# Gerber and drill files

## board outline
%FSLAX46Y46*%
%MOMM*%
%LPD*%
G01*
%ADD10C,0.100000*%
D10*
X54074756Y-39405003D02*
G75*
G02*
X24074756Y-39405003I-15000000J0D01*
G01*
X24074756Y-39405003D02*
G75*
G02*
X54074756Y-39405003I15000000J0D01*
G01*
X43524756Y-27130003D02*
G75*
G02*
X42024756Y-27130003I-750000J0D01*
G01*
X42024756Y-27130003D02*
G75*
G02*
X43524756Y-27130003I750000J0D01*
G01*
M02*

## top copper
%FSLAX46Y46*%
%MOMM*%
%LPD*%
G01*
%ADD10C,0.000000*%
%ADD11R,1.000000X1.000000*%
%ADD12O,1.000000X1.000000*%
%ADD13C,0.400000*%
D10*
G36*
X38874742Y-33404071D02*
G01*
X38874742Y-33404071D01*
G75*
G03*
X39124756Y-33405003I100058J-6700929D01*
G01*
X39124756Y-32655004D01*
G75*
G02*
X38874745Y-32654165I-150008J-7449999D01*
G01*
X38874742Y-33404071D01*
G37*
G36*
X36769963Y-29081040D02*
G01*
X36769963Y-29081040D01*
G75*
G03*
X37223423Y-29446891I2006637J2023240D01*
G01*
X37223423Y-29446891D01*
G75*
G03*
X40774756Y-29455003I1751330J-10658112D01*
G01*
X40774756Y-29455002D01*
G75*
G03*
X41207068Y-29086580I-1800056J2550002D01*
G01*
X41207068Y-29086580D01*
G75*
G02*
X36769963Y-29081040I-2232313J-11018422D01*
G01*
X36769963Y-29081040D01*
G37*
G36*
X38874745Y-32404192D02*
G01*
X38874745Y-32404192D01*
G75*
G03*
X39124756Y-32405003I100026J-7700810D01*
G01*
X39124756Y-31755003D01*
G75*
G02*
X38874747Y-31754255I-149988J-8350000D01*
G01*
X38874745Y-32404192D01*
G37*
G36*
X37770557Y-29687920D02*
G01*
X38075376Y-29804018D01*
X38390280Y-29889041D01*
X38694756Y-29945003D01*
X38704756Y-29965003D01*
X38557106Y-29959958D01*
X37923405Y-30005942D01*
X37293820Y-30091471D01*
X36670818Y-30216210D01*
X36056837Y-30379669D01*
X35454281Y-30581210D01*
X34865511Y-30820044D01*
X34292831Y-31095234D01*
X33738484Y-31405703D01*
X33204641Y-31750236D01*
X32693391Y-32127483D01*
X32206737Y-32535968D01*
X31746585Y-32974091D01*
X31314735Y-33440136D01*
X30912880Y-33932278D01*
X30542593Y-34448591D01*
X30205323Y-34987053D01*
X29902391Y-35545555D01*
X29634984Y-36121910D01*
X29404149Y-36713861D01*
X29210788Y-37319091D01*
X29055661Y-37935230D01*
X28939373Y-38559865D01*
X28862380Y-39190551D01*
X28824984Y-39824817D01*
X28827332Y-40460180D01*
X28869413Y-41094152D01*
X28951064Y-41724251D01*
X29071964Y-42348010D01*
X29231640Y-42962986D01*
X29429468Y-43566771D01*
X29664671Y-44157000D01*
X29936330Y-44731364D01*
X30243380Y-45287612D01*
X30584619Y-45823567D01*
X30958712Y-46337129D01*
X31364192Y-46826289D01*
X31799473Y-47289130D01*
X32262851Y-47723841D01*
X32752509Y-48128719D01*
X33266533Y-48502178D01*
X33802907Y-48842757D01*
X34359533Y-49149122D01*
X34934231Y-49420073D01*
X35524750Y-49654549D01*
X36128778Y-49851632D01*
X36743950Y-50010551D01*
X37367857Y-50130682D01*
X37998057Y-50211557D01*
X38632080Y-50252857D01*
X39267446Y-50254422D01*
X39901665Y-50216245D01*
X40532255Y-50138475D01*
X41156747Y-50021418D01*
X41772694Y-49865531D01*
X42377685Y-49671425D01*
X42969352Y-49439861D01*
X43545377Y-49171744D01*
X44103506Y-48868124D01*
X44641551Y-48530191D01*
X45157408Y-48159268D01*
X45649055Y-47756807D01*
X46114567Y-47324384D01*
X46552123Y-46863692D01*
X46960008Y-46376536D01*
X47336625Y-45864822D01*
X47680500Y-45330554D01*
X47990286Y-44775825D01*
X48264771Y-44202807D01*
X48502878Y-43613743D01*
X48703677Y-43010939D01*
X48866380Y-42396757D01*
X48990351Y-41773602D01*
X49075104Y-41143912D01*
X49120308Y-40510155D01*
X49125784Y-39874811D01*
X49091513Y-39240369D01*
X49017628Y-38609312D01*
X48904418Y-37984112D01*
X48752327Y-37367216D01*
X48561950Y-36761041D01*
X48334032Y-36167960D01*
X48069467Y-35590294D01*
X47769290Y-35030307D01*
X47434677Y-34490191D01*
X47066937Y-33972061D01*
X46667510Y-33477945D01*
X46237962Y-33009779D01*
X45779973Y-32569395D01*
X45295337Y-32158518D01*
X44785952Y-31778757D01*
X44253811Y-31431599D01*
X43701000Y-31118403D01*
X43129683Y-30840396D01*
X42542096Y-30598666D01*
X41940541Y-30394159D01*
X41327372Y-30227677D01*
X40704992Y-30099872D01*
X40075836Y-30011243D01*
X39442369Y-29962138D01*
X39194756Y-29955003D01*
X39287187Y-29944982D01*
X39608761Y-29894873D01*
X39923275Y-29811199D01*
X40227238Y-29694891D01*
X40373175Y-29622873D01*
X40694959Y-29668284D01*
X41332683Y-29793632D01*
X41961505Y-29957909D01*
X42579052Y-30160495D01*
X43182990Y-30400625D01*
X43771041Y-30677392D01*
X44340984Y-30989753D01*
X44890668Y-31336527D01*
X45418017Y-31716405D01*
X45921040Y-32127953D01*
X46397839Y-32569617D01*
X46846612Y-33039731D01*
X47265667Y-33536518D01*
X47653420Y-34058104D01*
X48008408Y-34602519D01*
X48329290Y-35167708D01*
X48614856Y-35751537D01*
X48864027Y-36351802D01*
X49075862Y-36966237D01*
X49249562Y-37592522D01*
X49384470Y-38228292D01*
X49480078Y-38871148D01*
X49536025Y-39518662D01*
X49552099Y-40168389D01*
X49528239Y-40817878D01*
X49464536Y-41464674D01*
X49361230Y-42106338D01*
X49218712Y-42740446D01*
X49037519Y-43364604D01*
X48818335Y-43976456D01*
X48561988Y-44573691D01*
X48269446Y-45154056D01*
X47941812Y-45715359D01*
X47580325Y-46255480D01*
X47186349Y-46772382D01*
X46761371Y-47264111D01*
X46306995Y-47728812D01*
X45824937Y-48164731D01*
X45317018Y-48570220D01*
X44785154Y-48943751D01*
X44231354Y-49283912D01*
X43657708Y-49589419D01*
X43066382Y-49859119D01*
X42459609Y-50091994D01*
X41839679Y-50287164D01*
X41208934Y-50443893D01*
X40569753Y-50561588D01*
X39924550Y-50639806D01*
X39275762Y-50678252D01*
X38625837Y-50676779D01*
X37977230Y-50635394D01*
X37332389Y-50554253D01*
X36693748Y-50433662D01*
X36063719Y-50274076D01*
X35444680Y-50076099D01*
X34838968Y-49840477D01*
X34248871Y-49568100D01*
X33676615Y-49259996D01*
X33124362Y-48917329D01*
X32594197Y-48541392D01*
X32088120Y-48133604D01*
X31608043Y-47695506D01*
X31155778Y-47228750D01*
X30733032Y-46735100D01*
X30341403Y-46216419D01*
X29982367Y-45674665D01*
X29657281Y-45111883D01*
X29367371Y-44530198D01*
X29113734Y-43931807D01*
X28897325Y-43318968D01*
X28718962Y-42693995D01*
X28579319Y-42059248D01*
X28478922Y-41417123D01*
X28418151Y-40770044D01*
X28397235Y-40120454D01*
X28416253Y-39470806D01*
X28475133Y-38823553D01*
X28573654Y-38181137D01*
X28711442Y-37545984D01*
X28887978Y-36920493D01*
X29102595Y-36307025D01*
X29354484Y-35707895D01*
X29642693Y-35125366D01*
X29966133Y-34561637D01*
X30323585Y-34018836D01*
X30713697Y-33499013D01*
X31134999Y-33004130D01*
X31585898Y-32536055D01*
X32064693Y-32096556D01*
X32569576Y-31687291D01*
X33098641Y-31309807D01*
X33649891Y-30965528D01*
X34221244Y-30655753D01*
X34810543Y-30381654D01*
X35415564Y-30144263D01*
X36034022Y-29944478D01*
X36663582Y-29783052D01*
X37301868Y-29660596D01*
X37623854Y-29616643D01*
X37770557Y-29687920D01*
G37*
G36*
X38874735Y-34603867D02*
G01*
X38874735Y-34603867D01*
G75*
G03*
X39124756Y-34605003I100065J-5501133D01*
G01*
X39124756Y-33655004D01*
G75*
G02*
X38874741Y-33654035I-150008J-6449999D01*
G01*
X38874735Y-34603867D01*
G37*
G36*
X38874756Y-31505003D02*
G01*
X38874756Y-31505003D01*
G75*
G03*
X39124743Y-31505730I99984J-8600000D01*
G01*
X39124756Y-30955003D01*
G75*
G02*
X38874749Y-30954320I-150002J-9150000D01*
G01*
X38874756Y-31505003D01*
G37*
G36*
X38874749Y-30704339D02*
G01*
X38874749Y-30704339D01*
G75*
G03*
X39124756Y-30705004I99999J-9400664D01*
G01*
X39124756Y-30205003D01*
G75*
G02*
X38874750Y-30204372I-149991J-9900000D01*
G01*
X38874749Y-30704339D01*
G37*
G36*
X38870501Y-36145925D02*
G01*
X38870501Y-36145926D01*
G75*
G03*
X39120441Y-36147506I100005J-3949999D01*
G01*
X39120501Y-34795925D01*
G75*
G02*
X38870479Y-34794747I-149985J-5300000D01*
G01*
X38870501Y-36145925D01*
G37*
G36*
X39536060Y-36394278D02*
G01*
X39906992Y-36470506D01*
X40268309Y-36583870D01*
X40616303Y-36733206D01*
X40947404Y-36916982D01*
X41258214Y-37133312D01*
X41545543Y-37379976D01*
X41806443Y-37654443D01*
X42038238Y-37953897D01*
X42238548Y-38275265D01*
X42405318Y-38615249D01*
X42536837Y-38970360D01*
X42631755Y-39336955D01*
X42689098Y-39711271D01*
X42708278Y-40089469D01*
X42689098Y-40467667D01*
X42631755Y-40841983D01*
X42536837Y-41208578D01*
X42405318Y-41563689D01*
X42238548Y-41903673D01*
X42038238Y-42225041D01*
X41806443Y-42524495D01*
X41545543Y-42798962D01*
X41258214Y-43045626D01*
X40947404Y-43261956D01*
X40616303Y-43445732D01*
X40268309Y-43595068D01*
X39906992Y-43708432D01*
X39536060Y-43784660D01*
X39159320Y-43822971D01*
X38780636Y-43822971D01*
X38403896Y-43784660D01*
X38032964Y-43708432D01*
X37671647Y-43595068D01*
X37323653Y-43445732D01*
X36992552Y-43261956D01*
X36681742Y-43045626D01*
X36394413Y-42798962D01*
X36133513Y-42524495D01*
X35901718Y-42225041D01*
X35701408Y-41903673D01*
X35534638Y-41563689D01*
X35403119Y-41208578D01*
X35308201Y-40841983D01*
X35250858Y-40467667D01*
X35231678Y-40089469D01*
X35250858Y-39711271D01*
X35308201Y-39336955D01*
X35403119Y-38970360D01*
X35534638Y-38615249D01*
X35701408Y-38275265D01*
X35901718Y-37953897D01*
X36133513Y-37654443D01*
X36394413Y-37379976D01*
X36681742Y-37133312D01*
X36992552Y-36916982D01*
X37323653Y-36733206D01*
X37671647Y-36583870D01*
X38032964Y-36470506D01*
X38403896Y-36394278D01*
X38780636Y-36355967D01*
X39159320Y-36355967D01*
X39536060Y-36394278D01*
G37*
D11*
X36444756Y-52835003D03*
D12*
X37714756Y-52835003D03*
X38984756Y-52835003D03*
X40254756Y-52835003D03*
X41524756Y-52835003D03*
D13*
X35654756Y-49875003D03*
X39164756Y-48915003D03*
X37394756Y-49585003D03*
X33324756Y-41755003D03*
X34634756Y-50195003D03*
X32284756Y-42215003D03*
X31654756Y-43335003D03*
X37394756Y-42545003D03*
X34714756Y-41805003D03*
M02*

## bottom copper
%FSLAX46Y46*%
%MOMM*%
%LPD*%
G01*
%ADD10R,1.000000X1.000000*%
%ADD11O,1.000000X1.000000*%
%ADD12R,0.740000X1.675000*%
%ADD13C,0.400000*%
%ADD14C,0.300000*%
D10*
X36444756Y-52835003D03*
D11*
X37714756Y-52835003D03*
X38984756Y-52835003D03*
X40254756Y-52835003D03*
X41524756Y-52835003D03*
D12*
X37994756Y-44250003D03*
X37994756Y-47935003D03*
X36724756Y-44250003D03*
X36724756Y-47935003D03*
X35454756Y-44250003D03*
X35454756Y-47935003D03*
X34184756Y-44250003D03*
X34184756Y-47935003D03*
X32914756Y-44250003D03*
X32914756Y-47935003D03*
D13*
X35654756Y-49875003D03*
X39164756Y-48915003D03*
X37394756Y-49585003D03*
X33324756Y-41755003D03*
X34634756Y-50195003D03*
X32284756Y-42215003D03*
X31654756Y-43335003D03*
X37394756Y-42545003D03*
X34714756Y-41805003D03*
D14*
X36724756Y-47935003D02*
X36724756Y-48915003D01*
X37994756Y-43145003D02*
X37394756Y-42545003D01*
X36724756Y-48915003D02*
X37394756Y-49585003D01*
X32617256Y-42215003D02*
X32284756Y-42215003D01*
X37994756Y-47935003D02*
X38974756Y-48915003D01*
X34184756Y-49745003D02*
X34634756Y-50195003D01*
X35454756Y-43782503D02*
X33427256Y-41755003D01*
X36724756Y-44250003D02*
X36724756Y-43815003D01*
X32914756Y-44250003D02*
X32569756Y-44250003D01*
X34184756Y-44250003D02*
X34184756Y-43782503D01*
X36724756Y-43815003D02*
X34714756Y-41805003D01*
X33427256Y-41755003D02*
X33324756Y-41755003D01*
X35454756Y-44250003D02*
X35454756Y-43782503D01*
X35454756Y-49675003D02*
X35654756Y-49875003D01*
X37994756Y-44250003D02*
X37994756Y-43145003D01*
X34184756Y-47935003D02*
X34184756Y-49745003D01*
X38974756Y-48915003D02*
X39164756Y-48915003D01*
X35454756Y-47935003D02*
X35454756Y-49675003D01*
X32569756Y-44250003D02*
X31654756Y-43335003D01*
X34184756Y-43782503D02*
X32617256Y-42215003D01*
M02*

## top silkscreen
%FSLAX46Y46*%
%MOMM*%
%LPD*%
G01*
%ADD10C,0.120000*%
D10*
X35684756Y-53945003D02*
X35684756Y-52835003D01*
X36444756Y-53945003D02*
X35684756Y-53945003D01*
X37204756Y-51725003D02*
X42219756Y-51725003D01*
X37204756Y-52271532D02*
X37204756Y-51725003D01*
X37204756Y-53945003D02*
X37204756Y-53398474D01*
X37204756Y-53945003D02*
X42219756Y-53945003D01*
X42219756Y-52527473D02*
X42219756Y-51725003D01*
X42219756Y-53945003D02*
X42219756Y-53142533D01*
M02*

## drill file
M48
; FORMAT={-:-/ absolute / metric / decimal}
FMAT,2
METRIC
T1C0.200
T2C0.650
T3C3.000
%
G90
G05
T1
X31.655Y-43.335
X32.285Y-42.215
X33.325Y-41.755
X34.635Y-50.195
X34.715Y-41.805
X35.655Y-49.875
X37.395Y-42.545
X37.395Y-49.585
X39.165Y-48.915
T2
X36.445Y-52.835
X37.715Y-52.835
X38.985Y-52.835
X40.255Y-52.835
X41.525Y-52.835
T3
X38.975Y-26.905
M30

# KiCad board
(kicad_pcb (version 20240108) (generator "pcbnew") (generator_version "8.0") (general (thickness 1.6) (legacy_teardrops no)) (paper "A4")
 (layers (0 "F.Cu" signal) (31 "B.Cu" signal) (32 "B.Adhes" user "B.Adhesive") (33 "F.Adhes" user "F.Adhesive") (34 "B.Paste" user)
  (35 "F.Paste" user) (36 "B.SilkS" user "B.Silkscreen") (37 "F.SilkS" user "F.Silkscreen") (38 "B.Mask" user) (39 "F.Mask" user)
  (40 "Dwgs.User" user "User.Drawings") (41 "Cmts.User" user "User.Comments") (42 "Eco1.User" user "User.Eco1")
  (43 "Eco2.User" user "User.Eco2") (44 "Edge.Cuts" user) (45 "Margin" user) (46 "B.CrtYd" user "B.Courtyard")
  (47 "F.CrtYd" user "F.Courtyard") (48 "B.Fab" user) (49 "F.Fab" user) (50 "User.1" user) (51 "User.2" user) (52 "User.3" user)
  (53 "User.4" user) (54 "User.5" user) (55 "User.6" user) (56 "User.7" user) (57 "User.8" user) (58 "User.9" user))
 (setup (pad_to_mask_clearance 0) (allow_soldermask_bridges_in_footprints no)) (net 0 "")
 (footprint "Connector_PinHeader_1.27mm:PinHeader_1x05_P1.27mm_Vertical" (layer "F.Cu") (at 36.444756 52.835003 90)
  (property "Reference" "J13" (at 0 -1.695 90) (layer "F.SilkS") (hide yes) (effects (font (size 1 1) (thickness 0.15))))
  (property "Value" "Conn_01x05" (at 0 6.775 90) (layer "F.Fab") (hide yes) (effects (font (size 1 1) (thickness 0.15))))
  (fp_line (start -1.11 -0.76) (end 0 -0.76) (stroke (width 0.12) (type solid)) (layer "F.SilkS"))
  (fp_line (start -1.11 0) (end -1.11 -0.76) (stroke (width 0.12) (type solid)) (layer "F.SilkS"))
  (fp_line (start 1.11 0.76) (end 1.11 5.775) (stroke (width 0.12) (type solid)) (layer "F.SilkS"))
  (fp_line (start 0.563471 0.76) (end 1.11 0.76) (stroke (width 0.12) (type solid)) (layer "F.SilkS"))
  (fp_line (start -1.11 0.76) (end -0.563471 0.76) (stroke (width 0.12) (type solid)) (layer "F.SilkS"))
  (fp_line (start -1.11 0.76) (end -1.11 5.775) (stroke (width 0.12) (type solid)) (layer "F.SilkS"))
  (fp_line (start 0.30753 5.775) (end 1.11 5.775) (stroke (width 0.12) (type solid)) (layer "F.SilkS"))
  (fp_line (start -1.11 5.775) (end -0.30753 5.775) (stroke (width 0.12) (type solid)) (layer "F.SilkS"))
  (pad "1" thru_hole rect (at 0 0 90) (size 1 1) (drill 0.65) (layers "*.Cu" "*.Mask") (remove_unused_layers no))
  (pad "2" thru_hole oval (at 0 1.27 90) (size 1 1) (drill 0.65) (layers "*.Cu" "*.Mask") (remove_unused_layers no))
  (pad "3" thru_hole oval (at 0 2.54 90) (size 1 1) (drill 0.65) (layers "*.Cu" "*.Mask") (remove_unused_layers no))
  (pad "4" thru_hole oval (at 0 3.81 90) (size 1 1) (drill 0.65) (layers "*.Cu" "*.Mask") (remove_unused_layers no))
  (pad "5" thru_hole oval (at 0 5.08 90) (size 1 1) (drill 0.65) (layers "*.Cu" "*.Mask") (remove_unused_layers no)))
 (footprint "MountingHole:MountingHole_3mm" (layer "F.Cu") (at 38.974756 26.905003)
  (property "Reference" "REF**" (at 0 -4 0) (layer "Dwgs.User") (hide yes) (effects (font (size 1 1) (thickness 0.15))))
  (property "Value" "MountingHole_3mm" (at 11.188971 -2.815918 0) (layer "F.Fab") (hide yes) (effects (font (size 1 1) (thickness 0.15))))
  (pad "" np_thru_hole circle (at 0 0) (size 3 3) (drill 3) (layers "*.Cu" "*.Mask")))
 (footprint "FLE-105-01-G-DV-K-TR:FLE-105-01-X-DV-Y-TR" (layer "B.Cu") (at 35.454756 46.092503 180)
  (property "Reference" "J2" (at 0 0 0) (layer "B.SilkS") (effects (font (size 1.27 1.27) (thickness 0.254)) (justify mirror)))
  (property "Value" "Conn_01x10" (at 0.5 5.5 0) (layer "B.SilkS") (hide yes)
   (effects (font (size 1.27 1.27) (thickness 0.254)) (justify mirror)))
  (pad "1" smd rect (at -2.54 1.8425 180) (size 0.74 1.675) (layers "B.Cu" "B.Paste" "B.Mask"))
  (pad "2" smd rect (at -2.54 -1.8425 180) (size 0.74 1.675) (layers "B.Cu" "B.Paste" "B.Mask"))
  (pad "3" smd rect (at -1.27 1.8425 180) (size 0.74 1.675) (layers "B.Cu" "B.Paste" "B.Mask"))
  (pad "4" smd rect (at -1.27 -1.8425 180) (size 0.74 1.675) (layers "B.Cu" "B.Paste" "B.Mask"))
  (pad "5" smd rect (at 0 1.8425 180) (size 0.74 1.675) (layers "B.Cu" "B.Paste" "B.Mask"))
  (pad "6" smd rect (at 0 -1.8425 180) (size 0.74 1.675) (layers "B.Cu" "B.Paste" "B.Mask"))
  (pad "7" smd rect (at 1.27 1.8425 180) (size 0.74 1.675) (layers "B.Cu" "B.Paste" "B.Mask"))
  (pad "8" smd rect (at 1.27 -1.8425 180) (size 0.74 1.675) (layers "B.Cu" "B.Paste" "B.Mask"))
  (pad "9" smd rect (at 2.54 1.8425 180) (size 0.74 1.675) (layers "B.Cu" "B.Paste" "B.Mask"))
  (pad "10" smd rect (at 2.54 -1.8425 180) (size 0.74 1.675) (layers "B.Cu" "B.Paste" "B.Mask")))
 (gr_poly
  (pts
   (arc (start 38.874745 32.654165) (mid 38.949758 47.55647) (end 39.124756 32.655004))
   (arc (start 39.124756 33.405003) (mid 38.949789 46.806633) (end 38.874742 33.404071)))
  (stroke (width 0) (type solid)) (fill solid) (layer "F.Cu"))
 (gr_poly
  (pts
   (arc (start 37.223423 29.446891) (mid 38.950087 50.906016) (end 40.774756 29.455003))
   (arc (start 40.774756 29.455002) (mid 40.99931 29.280645) (end 41.207068 29.08658))
   (arc (start 41.207068 29.08658) (mid 38.960716 51.347273) (end 36.769963 29.08104))
   (arc (start 36.769963 29.08104) (mid 36.987318 29.275586) (end 37.223423 29.446891)))
  (stroke (width 0) (type solid)) (fill solid) (layer "F.Cu"))
 (gr_poly
  (pts
   (arc (start 38.874745 32.404192) (mid 38.949788 47.806421) (end 39.124756 32.405003))
   (arc (start 39.124756 31.755003) (mid 38.949758 48.456313) (end 38.874747 31.754255)))
  (stroke (width 0) (type solid)) (fill solid) (layer "F.Cu"))
 (gr_poly
  (pts (xy 39.194756 29.955003) (xy 39.287187 29.944982) (xy 39.608761 29.894873) (xy 39.923275 29.811199) (xy 40.227238 29.694891)
   (xy 40.373175 29.622873) (xy 40.694959 29.668284) (xy 41.332683 29.793632) (xy 41.961505 29.957909) (xy 42.579052 30.160495)
   (xy 43.18299 30.400625) (xy 43.771041 30.677392) (xy 44.340984 30.989753) (xy 44.890668 31.336527) (xy 45.418017 31.716405)
   (xy 45.92104 32.127953) (xy 46.397839 32.569617) (xy 46.846612 33.039731) (xy 47.265667 33.536518) (xy 47.65342 34.058104)
   (xy 48.008408 34.602519) (xy 48.32929 35.167708) (xy 48.614856 35.751537) (xy 48.864027 36.351802) (xy 49.075862 36.966237)
   (xy 49.249562 37.592522) (xy 49.38447 38.228292) (xy 49.480078 38.871148) (xy 49.536025 39.518662) (xy 49.552099 40.168389)
   (xy 49.528239 40.817878) (xy 49.464536 41.464674) (xy 49.36123 42.106338) (xy 49.218712 42.740446) (xy 49.037519 43.364604)
   (xy 48.818335 43.976456) (xy 48.561988 44.573691) (xy 48.269446 45.154056) (xy 47.941812 45.715359) (xy 47.580325 46.25548)
   (xy 47.186349 46.772382) (xy 46.761371 47.264111) (xy 46.306995 47.728812) (xy 45.824937 48.164731) (xy 45.317018 48.57022)
   (xy 44.785154 48.943751) (xy 44.231354 49.283912) (xy 43.657708 49.589419) (xy 43.066382 49.859119) (xy 42.459609 50.091994)
   (xy 41.839679 50.287164) (xy 41.208934 50.443893) (xy 40.569753 50.561588) (xy 39.92455 50.639806) (xy 39.275762 50.678252)
   (xy 38.625837 50.676779) (xy 37.97723 50.635394) (xy 37.332389 50.554253) (xy 36.693748 50.433662) (xy 36.063719 50.274076)
   (xy 35.44468 50.076099) (xy 34.838968 49.840477) (xy 34.248871 49.5681) (xy 33.676615 49.259996) (xy 33.124362 48.917329)
   (xy 32.594197 48.541392) (xy 32.08812 48.133604) (xy 31.608043 47.695506) (xy 31.155778 47.22875) (xy 30.733032 46.7351)
   (xy 30.341403 46.216419) (xy 29.982367 45.674665) (xy 29.657281 45.111883) (xy 29.367371 44.530198) (xy 29.113734 43.931807)
   (xy 28.897325 43.318968) (xy 28.718962 42.693995) (xy 28.579319 42.059248) (xy 28.478922 41.417123) (xy 28.418151 40.770044)
   (xy 28.397235 40.120454) (xy 28.416253 39.470806) (xy 28.475133 38.823553) (xy 28.573654 38.181137) (xy 28.711442 37.545984)
   (xy 28.887978 36.920493) (xy 29.102595 36.307025) (xy 29.354484 35.707895) (xy 29.642693 35.125366) (xy 29.966133 34.561637)
   (xy 30.323585 34.018836) (xy 30.713697 33.499013) (xy 31.134999 33.00413) (xy 31.585898 32.536055) (xy 32.064693 32.096556)
   (xy 32.569576 31.687291) (xy 33.098641 31.309807) (xy 33.649891 30.965528) (xy 34.221244 30.655753) (xy 34.810543 30.381654)
   (xy 35.415564 30.144263) (xy 36.034022 29.944478) (xy 36.663582 29.783052) (xy 37.301868 29.660596) (xy 37.623854 29.616643)
   (xy 37.770557 29.68792) (xy 38.075376 29.804018) (xy 38.39028 29.889041) (xy 38.694756 29.945003) (xy 38.704756 29.965003)
   (xy 38.557106 29.959958) (xy 37.923405 30.005942) (xy 37.29382 30.091471) (xy 36.670818 30.21621) (xy 36.056837 30.379669)
   (xy 35.454281 30.58121) (xy 34.865511 30.820044) (xy 34.292831 31.095234) (xy 33.738484 31.405703) (xy 33.204641 31.750236)
   (xy 32.693391 32.127483) (xy 32.206737 32.535968) (xy 31.746585 32.974091) (xy 31.314735 33.440136) (xy 30.91288 33.932278)
   (xy 30.542593 34.448591) (xy 30.205323 34.987053) (xy 29.902391 35.545555) (xy 29.634984 36.12191) (xy 29.404149 36.713861)
   (xy 29.210788 37.319091) (xy 29.055661 37.93523) (xy 28.939373 38.559865) (xy 28.86238 39.190551) (xy 28.824984 39.824817)
   (xy 28.827332 40.46018) (xy 28.869413 41.094152) (xy 28.951064 41.724251) (xy 29.071964 42.34801) (xy 29.23164 42.962986)
   (xy 29.429468 43.566771) (xy 29.664671 44.157) (xy 29.93633 44.731364) (xy 30.24338 45.287612) (xy 30.584619 45.823567)
   (xy 30.958712 46.337129) (xy 31.364192 46.826289) (xy 31.799473 47.28913) (xy 32.262851 47.723841) (xy 32.752509 48.128719)
   (xy 33.266533 48.502178) (xy 33.802907 48.842757) (xy 34.359533 49.149122) (xy 34.934231 49.420073) (xy 35.52475 49.654549)
   (xy 36.128778 49.851632) (xy 36.74395 50.010551) (xy 37.367857 50.130682) (xy 37.998057 50.211557) (xy 38.63208 50.252857)
   (xy 39.267446 50.254422) (xy 39.901665 50.216245) (xy 40.532255 50.138475) (xy 41.156747 50.021418) (xy 41.772694 49.865531)
   (xy 42.377685 49.671425) (xy 42.969352 49.439861) (xy 43.545377 49.171744) (xy 44.103506 48.868124) (xy 44.641551 48.530191)
   (xy 45.157408 48.159268) (xy 45.649055 47.756807) (xy 46.114567 47.324384) (xy 46.552123 46.863692) (xy 46.960008 46.376536)
   (xy 47.336625 45.864822) (xy 47.6805 45.330554) (xy 47.990286 44.775825) (xy 48.264771 44.202807) (xy 48.502878 43.613743)
   (xy 48.703677 43.010939) (xy 48.86638 42.396757) (xy 48.990351 41.773602) (xy 49.075104 41.143912) (xy 49.120308 40.510155)
   (xy 49.125784 39.874811) (xy 49.091513 39.240369) (xy 49.017628 38.609312) (xy 48.904418 37.984112) (xy 48.752327 37.367216)
   (xy 48.56195 36.761041) (xy 48.334032 36.16796) (xy 48.069467 35.590294) (xy 47.76929 35.030307) (xy 47.434677 34.490191)
   (xy 47.066937 33.972061) (xy 46.66751 33.477945) (xy 46.237962 33.009779) (xy 45.779973 32.569395) (xy 45.295337 32.158518)
   (xy 44.785952 31.778757) (xy 44.253811 31.431599) (xy 43.701 31.118403) (xy 43.129683 30.840396) (xy 42.542096 30.598666)
   (xy 41.940541 30.394159) (xy 41.327372 30.227677) (xy 40.704992 30.099872) (xy 40.075836 30.011243) (xy 39.442369 29.962138))
  (stroke (width 0) (type solid)) (fill solid) (layer "F.Cu"))
 (gr_poly
  (pts (xy 39.124756 33.655003)
   (arc (start 39.124756 34.605003) (mid 38.94976 45.606991) (end 38.874735 34.603867))
   (arc (start 38.874741 33.654035) (mid 38.949759 46.556698) (end 39.124756 33.655004)))
  (stroke (width 0) (type solid)) (fill solid) (layer "F.Cu"))
 (gr_poly
  (pts
   (arc (start 38.874756 31.505003) (mid 38.94976 48.705548) (end 39.124743 31.50573))
   (arc (start 39.124756 30.955003) (mid 38.949757 49.256198) (end 38.874749 30.95432)))
  (stroke (width 0) (type solid)) (fill solid) (layer "F.Cu"))
 (gr_poly
  (pts
   (arc (start 38.874749 30.704339) (mid 38.949757 49.506165) (end 39.124756 30.705004))
   (arc (start 39.124756 30.205003) (mid 38.949757 50.006108) (end 38.87475 30.204372)))
  (stroke (width 0) (type solid)) (fill solid) (layer "F.Cu"))
 (gr_poly
  (pts
   (arc (start 38.870501 36.145926) (mid 38.945519 44.047111) (end 39.120441 36.147506))
   (arc (start 39.120501 34.795925) (mid 38.945505 45.397988) (end 38.870479 34.794747)) (xy 38.870501 36.145925))
  (stroke (width 0) (type solid)) (fill solid) (layer "F.Cu"))
 (gr_poly
  (pts (xy 42.708278 40.089469) (xy 42.689098 39.711271) (xy 42.631755 39.336955) (xy 42.536837 38.97036) (xy 42.405318 38.615249)
   (xy 42.238548 38.275265) (xy 42.038238 37.953897) (xy 41.806443 37.654443) (xy 41.545543 37.379976) (xy 41.258214 37.133312)
   (xy 40.947404 36.916982) (xy 40.616303 36.733206) (xy 40.268309 36.58387) (xy 39.906992 36.470506) (xy 39.53606 36.394278)
   (xy 39.15932 36.355967) (xy 38.780636 36.355967) (xy 38.403896 36.394278) (xy 38.032964 36.470506) (xy 37.671647 36.58387)
   (xy 37.323653 36.733206) (xy 36.992552 36.916982) (xy 36.681742 37.133312) (xy 36.394413 37.379976) (xy 36.133513 37.654443)
   (xy 35.901718 37.953897) (xy 35.701408 38.275265) (xy 35.534638 38.615249) (xy 35.403119 38.97036) (xy 35.308201 39.336955)
   (xy 35.250858 39.711271) (xy 35.231678 40.089469) (xy 35.250858 40.467667) (xy 35.308201 40.841983) (xy 35.403119 41.208578)
   (xy 35.534638 41.563689) (xy 35.701408 41.903673) (xy 35.901718 42.225041) (xy 36.133513 42.524495) (xy 36.394413 42.798962)
   (xy 36.681742 43.045626) (xy 36.992552 43.261956) (xy 37.323653 43.445732) (xy 37.671647 43.595068) (xy 38.032964 43.708432)
   (xy 38.403896 43.78466) (xy 38.780636 43.822971) (xy 39.15932 43.822971) (xy 39.53606 43.78466) (xy 39.906992 43.708432)
   (xy 40.268309 43.595068) (xy 40.616303 43.445732) (xy 40.947404 43.261956) (xy 41.258214 43.045626) (xy 41.545543 42.798962)
   (xy 41.806443 42.524495) (xy 42.038238 42.225041) (xy 42.238548 41.903673) (xy 42.405318 41.563689) (xy 42.536837 41.208578)
   (xy 42.631755 40.841983) (xy 42.689098 40.467667) (xy 42.708278 40.089469))
  (stroke (width 0) (type solid)) (fill solid) (layer "F.Cu"))
 (gr_circle (center 39.074756 39.405003) (end 54.074756 39.405003) (stroke (width 0.1) (type default)) (fill none) (layer "Edge.Cuts"))
 (gr_circle (center 42.774756 27.130003) (end 43.524756 27.130003) (stroke (width 0.1) (type default)) (fill none) (layer "Edge.Cuts"))
 (via (at 35.654756 49.875003) (size 0.4) (drill 0.2) (layers "F.Cu" "B.Cu") (remove_unused_layers yes) (keep_end_layers yes)
  (zone_layer_connections) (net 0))
 (via (at 39.164756 48.915003) (size 0.4) (drill 0.2) (layers "F.Cu" "B.Cu") (remove_unused_layers yes) (keep_end_layers yes)
  (zone_layer_connections) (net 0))
 (via (at 37.394756 49.585003) (size 0.4) (drill 0.2) (layers "F.Cu" "B.Cu") (remove_unused_layers yes) (keep_end_layers yes)
  (zone_layer_connections) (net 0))
 (via (at 33.324756 41.755003) (size 0.4) (drill 0.2) (layers "F.Cu" "B.Cu") (remove_unused_layers yes) (keep_end_layers yes)
  (zone_layer_connections) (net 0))
 (via (at 34.634756 50.195003) (size 0.4) (drill 0.2) (layers "F.Cu" "B.Cu") (remove_unused_layers yes) (keep_end_layers yes)
  (zone_layer_connections) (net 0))
 (via (at 32.284756 42.215003) (size 0.4) (drill 0.2) (layers "F.Cu" "B.Cu") (remove_unused_layers yes) (keep_end_layers yes)
  (zone_layer_connections) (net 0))
 (via (at 31.654756 43.335003) (size 0.4) (drill 0.2) (layers "F.Cu" "B.Cu") (remove_unused_layers yes) (keep_end_layers yes)
  (zone_layer_connections) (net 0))
 (via (at 37.394756 42.545003) (size 0.4) (drill 0.2) (layers "F.Cu" "B.Cu") (remove_unused_layers yes) (keep_end_layers yes)
  (zone_layer_connections) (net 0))
 (via (at 34.714756 41.805003) (size 0.4) (drill 0.2) (layers "F.Cu" "B.Cu") (remove_unused_layers yes) (keep_end_layers yes)
  (zone_layer_connections) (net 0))
 (segment (start 36.724756 47.935003) (end 36.724756 48.915003) (width 0.3) (layer "B.Cu") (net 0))
 (segment (start 37.994756 43.145003) (end 37.394756 42.545003) (width 0.3) (layer "B.Cu") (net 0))
 (segment (start 36.724756 48.915003) (end 37.394756 49.585003) (width 0.3) (layer "B.Cu") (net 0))
 (segment (start 32.617256 42.215003) (end 32.284756 42.215003) (width 0.3) (layer "B.Cu") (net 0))
 (segment (start 37.994756 47.935003) (end 38.974756 48.915003) (width 0.3) (layer "B.Cu") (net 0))
 (segment (start 34.184756 49.745003) (end 34.634756 50.195003) (width 0.3) (layer "B.Cu") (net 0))
 (segment (start 35.454756 43.782503) (end 33.427256 41.755003) (width 0.3) (layer "B.Cu") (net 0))
 (segment (start 36.724756 44.250003) (end 36.724756 43.815003) (width 0.3) (layer "B.Cu") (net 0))
 (segment (start 32.914756 44.250003) (end 32.569756 44.250003) (width 0.3) (layer "B.Cu") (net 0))
 (segment (start 34.184756 44.250003) (end 34.184756 43.782503) (width 0.3) (layer "B.Cu") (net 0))
 (segment (start 36.724756 43.815003) (end 34.714756 41.805003) (width 0.3) (layer "B.Cu") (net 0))
 (segment (start 33.427256 41.755003) (end 33.324756 41.755003) (width 0.3) (layer "B.Cu") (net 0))
 (segment (start 35.454756 44.250003) (end 35.454756 43.782503) (width 0.3) (layer "B.Cu") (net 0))
 (segment (start 35.454756 49.675003) (end 35.654756 49.875003) (width 0.3) (layer "B.Cu") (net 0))
 (segment (start 37.994756 44.250003) (end 37.994756 43.145003) (width 0.3) (layer "B.Cu") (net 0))
 (segment (start 34.184756 47.935003) (end 34.184756 49.745003) (width 0.3) (layer "B.Cu") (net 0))
 (segment (start 38.974756 48.915003) (end 39.164756 48.915003) (width 0.3) (layer "B.Cu") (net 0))
 (segment (start 35.454756 47.935003) (end 35.454756 49.675003) (width 0.3) (layer "B.Cu") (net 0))
 (segment (start 32.569756 44.250003) (end 31.654756 43.335003) (width 0.3) (layer "B.Cu") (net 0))
 (segment (start 34.184756 43.782503) (end 32.617256 42.215003) (width 0.3) (layer "B.Cu") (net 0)))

